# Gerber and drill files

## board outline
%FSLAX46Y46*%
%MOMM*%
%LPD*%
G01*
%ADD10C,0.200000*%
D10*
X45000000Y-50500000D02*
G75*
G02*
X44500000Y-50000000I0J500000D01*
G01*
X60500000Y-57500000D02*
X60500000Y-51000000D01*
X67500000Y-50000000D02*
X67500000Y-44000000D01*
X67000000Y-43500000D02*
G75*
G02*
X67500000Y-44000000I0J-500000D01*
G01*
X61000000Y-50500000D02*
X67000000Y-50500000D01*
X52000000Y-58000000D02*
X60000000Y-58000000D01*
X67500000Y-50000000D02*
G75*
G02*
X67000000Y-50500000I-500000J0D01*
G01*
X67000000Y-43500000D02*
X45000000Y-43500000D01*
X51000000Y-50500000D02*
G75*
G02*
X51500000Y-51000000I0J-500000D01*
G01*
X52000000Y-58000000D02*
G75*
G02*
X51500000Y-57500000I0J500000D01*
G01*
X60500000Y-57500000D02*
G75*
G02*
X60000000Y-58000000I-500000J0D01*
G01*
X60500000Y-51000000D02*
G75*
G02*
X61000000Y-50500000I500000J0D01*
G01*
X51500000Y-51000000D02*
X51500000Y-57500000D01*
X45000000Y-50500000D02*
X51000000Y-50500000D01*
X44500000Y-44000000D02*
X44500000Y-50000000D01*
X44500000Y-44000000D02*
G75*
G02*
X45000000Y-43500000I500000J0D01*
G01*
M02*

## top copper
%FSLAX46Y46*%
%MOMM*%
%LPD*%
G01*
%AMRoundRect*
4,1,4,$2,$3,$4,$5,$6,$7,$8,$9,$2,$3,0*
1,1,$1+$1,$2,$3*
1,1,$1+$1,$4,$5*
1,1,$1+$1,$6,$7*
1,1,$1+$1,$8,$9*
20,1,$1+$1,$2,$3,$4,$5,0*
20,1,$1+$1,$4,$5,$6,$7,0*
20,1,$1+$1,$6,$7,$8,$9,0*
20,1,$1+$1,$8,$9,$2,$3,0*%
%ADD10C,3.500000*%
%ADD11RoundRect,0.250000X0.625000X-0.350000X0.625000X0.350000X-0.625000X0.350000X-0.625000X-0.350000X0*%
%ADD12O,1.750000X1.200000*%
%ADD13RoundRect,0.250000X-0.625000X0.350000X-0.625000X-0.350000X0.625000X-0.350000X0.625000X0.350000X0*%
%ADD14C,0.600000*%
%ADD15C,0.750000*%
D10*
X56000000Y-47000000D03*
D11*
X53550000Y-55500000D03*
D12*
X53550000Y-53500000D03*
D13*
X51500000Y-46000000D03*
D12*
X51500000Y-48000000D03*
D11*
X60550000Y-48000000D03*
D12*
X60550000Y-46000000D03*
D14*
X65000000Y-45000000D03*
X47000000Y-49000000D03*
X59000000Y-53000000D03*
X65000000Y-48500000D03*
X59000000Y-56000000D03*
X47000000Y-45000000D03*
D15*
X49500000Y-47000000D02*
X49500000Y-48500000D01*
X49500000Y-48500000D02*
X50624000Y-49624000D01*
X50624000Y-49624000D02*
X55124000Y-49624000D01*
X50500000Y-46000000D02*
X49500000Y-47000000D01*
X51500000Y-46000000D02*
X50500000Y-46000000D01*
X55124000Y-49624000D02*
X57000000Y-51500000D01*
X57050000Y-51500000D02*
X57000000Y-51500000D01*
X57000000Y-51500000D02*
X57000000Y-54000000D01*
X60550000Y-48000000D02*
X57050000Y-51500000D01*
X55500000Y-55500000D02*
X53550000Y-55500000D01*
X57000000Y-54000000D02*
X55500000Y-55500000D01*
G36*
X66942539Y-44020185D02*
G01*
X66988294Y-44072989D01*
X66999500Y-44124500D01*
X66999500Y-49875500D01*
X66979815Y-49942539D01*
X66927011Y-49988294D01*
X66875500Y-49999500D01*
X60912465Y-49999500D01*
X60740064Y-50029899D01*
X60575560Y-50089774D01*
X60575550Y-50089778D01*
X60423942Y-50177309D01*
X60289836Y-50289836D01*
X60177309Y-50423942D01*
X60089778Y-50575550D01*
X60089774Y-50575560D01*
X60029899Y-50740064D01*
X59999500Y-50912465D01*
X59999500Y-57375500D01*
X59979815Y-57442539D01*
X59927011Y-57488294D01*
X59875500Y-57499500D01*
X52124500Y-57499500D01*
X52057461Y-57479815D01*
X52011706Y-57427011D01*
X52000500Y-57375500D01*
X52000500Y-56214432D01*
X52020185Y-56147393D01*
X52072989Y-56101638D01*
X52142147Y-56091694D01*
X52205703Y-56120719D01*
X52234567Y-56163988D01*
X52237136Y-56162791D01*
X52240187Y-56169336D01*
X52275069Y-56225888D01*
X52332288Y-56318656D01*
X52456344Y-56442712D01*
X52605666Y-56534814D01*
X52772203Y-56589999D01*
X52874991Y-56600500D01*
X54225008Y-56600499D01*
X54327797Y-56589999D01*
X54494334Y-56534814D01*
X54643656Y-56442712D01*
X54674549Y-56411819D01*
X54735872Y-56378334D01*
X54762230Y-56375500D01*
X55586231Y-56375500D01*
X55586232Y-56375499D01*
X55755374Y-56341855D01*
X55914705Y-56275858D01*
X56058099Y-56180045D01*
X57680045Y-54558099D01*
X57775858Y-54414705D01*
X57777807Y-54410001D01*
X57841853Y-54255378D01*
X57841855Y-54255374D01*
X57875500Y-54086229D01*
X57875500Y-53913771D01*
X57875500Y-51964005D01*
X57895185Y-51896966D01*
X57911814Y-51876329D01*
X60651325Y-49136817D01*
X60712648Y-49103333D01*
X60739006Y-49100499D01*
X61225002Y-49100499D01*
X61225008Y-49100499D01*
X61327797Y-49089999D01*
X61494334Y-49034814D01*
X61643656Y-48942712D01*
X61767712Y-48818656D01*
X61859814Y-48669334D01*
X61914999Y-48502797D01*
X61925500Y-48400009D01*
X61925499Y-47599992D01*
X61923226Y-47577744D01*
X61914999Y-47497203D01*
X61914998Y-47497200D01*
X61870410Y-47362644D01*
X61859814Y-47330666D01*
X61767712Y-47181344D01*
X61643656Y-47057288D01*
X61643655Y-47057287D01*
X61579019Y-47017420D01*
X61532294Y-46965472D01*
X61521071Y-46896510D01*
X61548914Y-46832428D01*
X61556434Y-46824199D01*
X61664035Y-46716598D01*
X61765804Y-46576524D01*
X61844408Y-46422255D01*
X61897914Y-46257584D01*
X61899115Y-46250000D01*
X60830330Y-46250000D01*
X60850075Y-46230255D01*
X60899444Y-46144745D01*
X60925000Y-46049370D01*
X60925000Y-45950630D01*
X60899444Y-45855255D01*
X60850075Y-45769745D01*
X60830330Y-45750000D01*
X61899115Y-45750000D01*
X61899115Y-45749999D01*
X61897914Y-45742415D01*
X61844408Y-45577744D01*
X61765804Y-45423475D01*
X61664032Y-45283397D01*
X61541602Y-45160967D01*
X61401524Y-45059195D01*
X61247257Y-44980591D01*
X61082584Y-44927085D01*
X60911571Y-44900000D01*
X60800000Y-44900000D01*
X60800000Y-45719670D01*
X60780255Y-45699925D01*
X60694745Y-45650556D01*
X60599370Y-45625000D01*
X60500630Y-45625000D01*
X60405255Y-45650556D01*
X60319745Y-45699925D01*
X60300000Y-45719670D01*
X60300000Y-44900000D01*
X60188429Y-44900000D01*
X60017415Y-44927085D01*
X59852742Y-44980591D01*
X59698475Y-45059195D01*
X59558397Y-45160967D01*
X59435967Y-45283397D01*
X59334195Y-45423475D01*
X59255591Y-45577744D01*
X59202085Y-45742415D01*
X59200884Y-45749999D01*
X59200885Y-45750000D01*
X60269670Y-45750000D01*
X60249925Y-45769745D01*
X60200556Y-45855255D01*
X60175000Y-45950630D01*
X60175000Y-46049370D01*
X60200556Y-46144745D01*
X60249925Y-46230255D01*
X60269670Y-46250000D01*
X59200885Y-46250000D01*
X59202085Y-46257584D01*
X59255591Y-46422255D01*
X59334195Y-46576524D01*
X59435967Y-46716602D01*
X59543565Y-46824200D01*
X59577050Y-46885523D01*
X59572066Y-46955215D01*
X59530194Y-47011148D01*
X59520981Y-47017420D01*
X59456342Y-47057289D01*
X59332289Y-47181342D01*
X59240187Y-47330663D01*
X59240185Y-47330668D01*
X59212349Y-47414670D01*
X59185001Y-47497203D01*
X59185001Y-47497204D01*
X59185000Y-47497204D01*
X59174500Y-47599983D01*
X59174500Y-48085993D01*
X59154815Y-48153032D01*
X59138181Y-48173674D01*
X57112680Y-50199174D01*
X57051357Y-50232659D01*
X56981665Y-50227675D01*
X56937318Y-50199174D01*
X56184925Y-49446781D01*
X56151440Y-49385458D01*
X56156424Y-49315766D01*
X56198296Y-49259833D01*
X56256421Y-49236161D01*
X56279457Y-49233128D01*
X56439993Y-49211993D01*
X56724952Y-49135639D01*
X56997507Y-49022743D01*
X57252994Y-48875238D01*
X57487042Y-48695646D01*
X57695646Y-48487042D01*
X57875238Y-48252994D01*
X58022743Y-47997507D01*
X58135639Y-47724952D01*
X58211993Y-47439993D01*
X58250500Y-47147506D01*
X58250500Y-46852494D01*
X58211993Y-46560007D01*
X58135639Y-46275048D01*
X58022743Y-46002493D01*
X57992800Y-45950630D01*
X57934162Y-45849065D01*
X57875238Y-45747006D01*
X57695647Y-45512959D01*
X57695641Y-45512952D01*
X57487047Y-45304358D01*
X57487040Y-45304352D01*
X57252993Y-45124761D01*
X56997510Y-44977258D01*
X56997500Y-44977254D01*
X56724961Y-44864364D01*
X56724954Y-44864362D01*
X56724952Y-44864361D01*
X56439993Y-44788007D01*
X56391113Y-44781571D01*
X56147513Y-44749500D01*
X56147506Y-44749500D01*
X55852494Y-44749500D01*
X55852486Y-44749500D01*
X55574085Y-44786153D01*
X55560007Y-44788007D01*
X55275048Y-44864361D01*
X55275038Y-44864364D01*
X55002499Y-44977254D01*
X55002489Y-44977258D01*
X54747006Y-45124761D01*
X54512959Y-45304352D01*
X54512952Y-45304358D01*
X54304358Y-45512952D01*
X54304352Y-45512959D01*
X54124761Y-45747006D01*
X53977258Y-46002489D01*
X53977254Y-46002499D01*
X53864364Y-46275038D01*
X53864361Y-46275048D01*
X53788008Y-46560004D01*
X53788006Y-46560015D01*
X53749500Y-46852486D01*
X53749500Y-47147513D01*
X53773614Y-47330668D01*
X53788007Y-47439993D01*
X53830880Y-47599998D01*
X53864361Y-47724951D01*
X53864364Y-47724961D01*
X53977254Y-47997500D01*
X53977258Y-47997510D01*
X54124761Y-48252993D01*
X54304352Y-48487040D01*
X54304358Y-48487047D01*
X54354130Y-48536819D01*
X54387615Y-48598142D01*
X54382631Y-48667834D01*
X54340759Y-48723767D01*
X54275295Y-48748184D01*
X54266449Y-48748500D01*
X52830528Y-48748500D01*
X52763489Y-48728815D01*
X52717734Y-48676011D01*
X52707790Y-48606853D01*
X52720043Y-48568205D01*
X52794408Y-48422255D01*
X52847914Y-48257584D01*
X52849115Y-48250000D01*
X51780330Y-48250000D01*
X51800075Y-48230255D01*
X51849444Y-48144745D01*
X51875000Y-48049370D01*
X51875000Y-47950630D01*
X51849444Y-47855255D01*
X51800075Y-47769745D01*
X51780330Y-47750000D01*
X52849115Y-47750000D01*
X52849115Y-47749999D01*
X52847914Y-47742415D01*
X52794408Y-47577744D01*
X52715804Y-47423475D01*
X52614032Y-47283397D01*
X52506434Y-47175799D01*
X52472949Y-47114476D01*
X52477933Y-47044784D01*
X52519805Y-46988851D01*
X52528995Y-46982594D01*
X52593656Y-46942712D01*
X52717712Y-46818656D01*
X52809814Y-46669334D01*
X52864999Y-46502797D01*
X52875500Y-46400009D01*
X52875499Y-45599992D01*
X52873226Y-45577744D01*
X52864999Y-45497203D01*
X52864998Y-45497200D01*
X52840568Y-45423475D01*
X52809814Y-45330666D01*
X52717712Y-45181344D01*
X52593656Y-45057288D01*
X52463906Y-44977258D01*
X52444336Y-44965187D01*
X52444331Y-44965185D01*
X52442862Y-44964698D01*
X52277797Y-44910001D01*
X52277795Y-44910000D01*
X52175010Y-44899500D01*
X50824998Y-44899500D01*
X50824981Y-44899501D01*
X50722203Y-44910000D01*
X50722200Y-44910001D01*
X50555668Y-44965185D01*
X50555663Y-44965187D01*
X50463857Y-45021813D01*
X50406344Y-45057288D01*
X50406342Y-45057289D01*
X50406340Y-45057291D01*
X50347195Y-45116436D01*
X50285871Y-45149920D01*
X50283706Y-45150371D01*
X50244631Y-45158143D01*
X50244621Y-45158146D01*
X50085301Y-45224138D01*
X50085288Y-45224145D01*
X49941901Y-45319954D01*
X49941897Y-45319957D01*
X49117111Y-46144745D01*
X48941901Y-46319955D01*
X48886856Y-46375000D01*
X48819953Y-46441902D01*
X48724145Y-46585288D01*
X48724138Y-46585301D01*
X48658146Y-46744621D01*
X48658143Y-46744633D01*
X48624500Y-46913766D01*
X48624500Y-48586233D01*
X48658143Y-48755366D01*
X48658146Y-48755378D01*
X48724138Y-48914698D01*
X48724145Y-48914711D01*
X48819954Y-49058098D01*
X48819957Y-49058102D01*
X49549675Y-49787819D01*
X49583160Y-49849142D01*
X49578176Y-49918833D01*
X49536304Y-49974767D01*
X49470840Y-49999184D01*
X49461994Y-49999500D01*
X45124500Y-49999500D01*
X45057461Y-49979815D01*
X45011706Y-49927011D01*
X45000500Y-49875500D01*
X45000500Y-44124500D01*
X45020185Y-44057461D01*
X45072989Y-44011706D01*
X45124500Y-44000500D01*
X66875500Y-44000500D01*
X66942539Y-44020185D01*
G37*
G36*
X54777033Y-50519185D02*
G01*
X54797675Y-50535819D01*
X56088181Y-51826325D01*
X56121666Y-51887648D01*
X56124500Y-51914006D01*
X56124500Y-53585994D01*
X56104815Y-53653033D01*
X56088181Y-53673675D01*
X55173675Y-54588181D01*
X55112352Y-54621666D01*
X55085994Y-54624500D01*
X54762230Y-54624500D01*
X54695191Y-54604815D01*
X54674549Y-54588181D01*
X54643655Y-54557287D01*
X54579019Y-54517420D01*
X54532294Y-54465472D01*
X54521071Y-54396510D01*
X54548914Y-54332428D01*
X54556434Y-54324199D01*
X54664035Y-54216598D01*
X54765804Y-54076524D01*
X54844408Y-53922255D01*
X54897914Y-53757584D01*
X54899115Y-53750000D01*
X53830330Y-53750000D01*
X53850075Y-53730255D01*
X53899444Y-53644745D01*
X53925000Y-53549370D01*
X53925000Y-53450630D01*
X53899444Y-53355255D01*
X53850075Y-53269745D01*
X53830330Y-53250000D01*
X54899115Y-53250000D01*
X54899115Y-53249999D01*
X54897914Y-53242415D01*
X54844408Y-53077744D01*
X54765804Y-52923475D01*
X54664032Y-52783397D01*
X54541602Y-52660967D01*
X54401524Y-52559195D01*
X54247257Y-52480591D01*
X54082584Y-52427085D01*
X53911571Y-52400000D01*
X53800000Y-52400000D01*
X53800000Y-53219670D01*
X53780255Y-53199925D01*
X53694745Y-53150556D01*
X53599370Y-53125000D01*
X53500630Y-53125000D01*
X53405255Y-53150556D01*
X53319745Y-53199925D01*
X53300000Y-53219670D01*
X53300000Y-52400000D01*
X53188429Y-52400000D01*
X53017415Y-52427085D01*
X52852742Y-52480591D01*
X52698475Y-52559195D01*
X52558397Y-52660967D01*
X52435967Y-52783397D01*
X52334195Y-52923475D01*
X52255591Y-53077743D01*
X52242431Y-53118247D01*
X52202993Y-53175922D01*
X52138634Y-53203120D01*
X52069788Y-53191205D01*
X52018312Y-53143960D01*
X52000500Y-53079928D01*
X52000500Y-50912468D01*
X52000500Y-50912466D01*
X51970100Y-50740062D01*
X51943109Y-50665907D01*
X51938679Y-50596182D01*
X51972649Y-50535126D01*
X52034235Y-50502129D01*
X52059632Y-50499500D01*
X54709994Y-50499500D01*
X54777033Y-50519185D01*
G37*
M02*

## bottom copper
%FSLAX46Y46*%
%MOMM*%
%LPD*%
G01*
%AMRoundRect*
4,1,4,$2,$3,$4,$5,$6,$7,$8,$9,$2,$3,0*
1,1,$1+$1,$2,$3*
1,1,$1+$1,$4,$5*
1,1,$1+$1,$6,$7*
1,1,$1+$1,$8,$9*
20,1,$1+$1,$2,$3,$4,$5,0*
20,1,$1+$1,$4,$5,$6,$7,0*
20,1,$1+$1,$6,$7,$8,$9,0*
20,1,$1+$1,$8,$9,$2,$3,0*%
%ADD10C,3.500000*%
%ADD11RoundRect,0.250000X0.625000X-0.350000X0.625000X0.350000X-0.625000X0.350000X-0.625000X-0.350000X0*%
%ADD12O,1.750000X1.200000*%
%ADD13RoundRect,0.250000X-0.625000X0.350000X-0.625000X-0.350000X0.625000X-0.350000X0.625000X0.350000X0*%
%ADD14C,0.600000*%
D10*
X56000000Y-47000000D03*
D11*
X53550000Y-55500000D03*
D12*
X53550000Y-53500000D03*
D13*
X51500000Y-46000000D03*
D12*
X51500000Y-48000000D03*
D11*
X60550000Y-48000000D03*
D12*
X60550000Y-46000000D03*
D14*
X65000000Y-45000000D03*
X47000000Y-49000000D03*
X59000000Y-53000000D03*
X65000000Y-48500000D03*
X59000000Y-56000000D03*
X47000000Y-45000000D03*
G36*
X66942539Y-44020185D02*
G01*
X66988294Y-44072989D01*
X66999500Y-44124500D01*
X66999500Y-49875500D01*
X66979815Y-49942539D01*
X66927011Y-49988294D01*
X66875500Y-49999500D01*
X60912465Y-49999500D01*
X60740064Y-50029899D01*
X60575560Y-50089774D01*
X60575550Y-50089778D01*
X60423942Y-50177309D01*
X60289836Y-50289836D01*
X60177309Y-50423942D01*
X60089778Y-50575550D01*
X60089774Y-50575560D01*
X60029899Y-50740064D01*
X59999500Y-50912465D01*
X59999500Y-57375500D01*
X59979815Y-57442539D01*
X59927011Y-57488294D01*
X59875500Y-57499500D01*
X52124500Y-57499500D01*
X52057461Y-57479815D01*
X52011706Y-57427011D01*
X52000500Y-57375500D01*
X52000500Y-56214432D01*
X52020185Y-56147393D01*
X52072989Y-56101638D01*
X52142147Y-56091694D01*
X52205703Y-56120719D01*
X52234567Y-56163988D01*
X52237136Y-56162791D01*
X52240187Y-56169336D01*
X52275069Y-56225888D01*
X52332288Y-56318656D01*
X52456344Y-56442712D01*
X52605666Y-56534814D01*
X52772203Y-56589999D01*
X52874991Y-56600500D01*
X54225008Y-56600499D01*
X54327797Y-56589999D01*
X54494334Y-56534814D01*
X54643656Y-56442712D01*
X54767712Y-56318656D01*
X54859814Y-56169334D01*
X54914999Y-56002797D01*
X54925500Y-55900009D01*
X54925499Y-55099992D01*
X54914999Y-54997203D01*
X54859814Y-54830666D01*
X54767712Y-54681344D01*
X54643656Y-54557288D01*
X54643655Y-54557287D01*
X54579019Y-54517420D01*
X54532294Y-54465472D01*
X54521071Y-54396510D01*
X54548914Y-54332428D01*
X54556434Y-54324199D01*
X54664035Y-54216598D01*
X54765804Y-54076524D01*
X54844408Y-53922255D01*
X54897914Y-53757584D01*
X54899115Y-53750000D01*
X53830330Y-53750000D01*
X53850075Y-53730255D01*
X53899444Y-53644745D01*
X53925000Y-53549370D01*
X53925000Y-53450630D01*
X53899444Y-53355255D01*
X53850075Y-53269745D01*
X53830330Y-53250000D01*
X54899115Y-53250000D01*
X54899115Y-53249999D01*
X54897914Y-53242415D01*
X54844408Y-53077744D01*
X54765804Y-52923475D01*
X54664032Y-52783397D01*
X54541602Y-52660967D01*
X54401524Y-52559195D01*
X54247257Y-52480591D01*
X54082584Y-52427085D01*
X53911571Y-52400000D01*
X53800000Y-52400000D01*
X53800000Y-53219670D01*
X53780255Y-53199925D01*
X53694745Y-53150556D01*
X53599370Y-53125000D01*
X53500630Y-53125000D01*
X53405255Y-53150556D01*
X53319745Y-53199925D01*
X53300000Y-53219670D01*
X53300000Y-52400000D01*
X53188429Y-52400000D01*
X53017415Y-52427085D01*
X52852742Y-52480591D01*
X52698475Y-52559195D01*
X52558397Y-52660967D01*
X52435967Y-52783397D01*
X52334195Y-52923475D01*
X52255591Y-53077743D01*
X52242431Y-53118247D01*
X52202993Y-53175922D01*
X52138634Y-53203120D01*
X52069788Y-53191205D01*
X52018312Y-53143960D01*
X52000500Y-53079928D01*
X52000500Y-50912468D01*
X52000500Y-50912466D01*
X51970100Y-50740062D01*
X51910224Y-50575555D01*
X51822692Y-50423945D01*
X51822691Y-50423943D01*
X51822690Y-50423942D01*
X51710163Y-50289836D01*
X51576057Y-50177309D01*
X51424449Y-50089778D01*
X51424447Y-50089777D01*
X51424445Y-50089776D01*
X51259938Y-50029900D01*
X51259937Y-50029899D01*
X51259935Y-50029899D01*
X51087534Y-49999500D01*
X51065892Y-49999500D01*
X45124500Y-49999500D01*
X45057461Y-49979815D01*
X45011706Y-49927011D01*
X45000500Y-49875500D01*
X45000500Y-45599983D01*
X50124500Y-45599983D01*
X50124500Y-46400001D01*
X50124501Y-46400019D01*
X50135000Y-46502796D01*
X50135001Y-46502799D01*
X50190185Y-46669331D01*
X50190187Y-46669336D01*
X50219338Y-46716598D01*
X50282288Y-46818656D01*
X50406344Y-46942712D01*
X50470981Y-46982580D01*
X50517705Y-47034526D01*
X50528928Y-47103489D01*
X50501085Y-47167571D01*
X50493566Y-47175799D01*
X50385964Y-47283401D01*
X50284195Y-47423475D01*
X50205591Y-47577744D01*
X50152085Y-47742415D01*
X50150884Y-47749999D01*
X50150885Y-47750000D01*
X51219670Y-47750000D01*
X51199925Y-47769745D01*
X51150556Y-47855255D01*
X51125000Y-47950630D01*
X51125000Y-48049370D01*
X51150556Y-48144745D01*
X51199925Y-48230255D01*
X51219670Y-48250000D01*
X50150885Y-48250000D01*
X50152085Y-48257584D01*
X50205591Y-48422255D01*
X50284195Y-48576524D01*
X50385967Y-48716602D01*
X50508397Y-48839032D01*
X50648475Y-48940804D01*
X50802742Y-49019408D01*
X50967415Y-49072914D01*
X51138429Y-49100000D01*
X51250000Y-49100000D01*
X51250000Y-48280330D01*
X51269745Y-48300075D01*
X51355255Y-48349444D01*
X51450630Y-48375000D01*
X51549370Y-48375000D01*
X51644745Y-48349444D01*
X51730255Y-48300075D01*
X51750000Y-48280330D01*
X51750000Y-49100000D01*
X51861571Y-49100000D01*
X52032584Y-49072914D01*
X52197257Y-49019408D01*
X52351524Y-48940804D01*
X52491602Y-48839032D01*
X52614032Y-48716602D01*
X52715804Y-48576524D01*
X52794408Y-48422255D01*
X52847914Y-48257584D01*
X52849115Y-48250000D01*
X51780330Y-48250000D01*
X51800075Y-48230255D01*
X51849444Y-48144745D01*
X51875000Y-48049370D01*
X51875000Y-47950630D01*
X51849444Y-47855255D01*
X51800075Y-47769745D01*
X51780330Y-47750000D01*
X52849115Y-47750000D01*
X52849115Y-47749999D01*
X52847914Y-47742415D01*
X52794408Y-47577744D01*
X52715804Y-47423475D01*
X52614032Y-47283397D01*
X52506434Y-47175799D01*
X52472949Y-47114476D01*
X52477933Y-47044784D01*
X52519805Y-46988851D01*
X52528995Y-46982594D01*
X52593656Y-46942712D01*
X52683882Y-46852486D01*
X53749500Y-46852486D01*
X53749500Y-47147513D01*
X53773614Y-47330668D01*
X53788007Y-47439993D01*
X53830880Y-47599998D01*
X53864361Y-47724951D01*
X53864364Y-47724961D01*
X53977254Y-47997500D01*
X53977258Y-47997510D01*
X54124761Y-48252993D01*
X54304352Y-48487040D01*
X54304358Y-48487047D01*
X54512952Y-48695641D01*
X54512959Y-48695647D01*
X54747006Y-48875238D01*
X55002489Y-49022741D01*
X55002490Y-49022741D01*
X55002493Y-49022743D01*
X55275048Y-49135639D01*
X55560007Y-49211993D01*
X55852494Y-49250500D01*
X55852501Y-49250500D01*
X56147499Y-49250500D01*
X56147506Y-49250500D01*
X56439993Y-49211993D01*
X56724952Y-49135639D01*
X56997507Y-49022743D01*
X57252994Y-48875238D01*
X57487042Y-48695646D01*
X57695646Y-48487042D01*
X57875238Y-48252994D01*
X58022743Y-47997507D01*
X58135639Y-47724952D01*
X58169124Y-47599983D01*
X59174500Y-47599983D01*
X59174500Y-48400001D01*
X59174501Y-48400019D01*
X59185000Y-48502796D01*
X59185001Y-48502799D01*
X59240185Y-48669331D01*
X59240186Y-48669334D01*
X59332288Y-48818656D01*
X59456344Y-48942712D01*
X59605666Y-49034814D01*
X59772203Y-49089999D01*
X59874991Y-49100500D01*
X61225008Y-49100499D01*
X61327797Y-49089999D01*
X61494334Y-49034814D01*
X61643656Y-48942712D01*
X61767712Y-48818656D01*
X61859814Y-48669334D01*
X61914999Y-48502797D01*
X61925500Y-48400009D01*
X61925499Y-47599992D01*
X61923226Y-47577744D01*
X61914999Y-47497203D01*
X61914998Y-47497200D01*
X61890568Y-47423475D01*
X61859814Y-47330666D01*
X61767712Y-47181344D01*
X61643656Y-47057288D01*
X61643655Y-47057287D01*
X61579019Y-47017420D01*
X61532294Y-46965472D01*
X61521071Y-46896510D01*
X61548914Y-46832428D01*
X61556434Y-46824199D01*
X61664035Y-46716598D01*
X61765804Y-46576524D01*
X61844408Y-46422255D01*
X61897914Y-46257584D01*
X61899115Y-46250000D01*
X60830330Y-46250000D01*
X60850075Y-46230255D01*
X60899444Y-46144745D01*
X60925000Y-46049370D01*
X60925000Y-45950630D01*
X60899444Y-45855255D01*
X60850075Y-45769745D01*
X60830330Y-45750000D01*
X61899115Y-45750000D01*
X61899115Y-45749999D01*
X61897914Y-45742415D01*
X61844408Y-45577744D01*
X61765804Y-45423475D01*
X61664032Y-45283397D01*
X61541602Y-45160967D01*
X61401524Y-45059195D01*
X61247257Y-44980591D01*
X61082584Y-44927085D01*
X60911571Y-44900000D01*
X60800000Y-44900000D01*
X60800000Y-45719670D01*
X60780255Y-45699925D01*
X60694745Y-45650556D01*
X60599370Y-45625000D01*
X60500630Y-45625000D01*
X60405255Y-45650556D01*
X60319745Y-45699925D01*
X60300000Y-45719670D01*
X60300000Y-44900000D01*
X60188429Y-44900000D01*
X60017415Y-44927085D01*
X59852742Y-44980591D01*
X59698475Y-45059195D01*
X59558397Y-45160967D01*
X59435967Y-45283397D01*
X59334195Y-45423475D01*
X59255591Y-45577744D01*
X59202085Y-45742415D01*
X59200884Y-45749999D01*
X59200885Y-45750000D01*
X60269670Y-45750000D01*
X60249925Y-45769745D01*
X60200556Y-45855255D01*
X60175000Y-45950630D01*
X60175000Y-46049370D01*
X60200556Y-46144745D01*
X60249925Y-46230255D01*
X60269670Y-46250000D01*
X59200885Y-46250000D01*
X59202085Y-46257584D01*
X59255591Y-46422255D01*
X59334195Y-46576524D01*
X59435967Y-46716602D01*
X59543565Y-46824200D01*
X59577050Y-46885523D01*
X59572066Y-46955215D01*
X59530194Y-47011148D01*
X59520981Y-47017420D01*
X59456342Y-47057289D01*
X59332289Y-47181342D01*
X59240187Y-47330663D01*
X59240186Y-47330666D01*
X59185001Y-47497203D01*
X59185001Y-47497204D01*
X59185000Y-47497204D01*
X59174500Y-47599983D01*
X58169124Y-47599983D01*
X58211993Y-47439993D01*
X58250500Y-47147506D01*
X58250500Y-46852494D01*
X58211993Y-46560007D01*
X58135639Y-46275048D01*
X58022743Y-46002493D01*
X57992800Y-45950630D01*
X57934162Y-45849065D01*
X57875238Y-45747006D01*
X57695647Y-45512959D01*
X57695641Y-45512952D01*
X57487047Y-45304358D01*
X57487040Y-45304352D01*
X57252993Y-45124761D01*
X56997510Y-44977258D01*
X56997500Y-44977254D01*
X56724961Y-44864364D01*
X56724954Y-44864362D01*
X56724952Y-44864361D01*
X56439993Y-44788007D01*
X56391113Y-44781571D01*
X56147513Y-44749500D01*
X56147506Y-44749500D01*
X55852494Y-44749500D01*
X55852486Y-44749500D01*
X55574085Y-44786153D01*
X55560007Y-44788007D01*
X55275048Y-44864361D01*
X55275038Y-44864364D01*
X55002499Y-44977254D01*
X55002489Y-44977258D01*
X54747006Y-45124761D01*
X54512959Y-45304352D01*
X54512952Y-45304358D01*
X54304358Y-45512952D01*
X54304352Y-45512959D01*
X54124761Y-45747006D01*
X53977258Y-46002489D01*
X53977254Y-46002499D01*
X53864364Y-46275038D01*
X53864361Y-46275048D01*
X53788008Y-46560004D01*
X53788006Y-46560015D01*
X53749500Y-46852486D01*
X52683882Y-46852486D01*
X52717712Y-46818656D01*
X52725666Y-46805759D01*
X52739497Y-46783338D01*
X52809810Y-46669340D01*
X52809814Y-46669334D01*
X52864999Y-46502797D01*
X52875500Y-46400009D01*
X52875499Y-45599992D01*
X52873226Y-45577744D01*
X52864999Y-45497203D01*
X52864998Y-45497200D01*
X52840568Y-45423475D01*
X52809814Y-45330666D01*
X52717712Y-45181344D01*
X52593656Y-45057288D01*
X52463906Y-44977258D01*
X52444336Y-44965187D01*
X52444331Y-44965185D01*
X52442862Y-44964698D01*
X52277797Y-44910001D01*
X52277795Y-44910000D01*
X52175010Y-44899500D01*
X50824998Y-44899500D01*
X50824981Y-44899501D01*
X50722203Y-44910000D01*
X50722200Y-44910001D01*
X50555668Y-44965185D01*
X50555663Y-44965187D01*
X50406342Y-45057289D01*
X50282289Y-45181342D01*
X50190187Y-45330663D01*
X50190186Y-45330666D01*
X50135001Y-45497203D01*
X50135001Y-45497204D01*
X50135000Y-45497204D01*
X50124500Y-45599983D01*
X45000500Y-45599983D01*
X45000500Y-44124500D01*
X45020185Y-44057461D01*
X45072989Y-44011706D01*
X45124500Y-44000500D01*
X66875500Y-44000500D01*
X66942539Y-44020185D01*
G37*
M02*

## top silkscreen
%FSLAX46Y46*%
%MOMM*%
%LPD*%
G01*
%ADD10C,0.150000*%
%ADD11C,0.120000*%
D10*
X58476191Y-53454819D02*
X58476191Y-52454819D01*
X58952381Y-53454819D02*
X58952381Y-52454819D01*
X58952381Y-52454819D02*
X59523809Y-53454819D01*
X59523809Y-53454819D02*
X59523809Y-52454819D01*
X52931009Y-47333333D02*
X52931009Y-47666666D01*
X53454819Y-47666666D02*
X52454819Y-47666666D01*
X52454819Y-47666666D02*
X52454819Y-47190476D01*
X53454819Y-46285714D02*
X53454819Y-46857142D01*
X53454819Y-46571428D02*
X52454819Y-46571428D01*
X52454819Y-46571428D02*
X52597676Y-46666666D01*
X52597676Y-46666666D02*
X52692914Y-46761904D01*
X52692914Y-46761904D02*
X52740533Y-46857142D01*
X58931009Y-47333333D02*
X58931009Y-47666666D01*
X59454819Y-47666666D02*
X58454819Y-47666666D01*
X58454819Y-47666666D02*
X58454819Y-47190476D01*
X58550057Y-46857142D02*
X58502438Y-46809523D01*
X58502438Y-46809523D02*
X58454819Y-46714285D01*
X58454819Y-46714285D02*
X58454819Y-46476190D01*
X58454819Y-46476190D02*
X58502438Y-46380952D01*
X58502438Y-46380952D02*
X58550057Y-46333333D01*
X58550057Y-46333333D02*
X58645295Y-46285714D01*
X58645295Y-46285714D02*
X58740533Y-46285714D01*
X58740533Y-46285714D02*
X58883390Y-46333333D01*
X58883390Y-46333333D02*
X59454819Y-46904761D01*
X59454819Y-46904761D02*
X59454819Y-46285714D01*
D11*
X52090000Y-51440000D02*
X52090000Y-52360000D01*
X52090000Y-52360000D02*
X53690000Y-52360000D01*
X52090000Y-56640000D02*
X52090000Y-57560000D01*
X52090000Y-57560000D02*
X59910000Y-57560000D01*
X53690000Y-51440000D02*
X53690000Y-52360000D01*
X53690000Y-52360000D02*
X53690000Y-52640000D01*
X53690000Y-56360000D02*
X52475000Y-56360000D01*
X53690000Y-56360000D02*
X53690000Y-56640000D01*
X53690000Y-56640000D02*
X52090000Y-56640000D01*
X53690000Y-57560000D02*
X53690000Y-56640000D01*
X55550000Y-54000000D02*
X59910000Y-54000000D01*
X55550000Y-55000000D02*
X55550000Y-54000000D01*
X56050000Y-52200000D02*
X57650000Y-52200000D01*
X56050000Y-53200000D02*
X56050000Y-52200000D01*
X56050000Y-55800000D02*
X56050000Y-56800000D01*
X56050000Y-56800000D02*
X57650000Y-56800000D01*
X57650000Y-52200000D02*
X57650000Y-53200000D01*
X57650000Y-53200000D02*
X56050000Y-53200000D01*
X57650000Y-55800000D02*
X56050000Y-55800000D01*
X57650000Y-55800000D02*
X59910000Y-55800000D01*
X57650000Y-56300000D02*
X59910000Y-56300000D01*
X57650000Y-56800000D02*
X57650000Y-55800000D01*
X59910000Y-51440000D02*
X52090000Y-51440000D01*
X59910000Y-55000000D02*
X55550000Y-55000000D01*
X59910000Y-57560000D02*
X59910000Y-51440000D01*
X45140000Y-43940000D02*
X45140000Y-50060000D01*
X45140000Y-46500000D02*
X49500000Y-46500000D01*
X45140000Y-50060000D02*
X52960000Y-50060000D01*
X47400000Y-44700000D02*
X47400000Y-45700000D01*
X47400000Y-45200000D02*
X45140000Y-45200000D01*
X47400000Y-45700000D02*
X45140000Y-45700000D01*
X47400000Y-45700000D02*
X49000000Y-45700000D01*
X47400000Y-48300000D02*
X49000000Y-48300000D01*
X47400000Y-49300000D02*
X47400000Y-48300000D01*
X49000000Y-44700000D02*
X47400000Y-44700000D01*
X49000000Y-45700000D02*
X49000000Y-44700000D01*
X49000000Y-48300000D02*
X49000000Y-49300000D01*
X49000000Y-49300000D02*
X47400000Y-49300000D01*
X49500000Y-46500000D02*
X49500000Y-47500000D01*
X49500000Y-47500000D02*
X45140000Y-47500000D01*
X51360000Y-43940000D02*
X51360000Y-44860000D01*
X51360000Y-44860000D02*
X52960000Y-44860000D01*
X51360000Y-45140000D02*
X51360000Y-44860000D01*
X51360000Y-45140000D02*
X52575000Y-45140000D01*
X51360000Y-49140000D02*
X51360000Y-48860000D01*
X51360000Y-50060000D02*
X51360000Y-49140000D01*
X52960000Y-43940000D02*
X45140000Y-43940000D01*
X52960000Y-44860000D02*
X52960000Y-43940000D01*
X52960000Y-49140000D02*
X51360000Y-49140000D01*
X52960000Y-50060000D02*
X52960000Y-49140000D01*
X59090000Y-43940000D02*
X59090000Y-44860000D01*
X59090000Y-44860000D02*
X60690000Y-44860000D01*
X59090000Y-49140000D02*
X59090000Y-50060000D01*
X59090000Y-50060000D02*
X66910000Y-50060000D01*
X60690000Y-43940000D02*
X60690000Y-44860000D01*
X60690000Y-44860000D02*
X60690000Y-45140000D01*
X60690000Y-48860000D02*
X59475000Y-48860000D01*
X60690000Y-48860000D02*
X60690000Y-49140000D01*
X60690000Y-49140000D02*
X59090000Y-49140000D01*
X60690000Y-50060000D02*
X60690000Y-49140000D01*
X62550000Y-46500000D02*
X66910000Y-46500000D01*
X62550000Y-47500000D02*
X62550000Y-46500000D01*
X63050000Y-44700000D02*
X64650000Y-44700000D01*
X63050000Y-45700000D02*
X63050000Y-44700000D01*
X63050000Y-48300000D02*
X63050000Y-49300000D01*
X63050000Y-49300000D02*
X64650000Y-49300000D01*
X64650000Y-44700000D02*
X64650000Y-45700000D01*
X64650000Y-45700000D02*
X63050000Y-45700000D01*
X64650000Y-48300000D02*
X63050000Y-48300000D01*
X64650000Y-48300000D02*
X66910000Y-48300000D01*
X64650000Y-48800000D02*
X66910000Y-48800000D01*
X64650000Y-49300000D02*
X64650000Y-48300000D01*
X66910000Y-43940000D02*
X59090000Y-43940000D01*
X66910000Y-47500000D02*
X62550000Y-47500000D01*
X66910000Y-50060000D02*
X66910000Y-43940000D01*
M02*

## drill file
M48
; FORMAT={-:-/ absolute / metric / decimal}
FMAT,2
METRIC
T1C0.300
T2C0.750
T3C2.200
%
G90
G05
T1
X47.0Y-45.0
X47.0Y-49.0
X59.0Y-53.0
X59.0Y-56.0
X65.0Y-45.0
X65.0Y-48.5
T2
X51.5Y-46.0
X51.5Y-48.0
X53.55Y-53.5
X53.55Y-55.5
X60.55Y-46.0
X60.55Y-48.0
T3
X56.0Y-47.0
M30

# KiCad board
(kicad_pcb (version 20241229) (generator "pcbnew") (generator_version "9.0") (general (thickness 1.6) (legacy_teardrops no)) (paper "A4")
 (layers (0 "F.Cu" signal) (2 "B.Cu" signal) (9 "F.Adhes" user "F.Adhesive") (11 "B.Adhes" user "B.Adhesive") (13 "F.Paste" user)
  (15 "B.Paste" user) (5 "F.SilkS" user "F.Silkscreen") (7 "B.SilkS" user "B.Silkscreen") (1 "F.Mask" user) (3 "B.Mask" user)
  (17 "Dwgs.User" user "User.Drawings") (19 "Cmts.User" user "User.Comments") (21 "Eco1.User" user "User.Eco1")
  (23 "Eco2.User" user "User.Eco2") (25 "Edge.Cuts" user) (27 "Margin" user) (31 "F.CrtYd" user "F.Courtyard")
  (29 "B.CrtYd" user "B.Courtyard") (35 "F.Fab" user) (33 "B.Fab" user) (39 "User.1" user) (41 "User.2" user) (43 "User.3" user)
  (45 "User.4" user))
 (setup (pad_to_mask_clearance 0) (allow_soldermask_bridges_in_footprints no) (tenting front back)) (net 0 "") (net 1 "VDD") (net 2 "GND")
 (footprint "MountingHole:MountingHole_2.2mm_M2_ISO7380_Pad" (layer "F.Cu") (at 56 47)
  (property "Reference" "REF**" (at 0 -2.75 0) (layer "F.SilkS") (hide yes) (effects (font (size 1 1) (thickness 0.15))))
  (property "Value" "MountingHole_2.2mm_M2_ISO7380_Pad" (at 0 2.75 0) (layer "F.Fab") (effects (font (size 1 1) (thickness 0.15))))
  (pad "1" thru_hole circle (at 0 0) (size 3.5 3.5) (drill 2.2) (layers "*.Cu" "*.Mask") (remove_unused_layers no)))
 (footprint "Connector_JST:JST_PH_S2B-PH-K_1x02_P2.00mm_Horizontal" (layer "F.Cu") (at 53.55 55.5 90)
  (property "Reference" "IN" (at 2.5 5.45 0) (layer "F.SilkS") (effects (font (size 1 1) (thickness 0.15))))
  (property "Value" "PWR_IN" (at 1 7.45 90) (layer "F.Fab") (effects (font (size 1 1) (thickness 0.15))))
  (fp_line (start 4.06 -1.46) (end 3.14 -1.46) (stroke (width 0.12) (type solid)) (layer "F.SilkS"))
  (fp_line (start 3.14 -1.46) (end 3.14 0.14) (stroke (width 0.12) (type solid)) (layer "F.SilkS"))
  (fp_line (start -1.14 -1.46) (end -2.06 -1.46) (stroke (width 0.12) (type solid)) (layer "F.SilkS"))
  (fp_line (start -2.06 -1.46) (end -2.06 6.36) (stroke (width 0.12) (type solid)) (layer "F.SilkS"))
  (fp_line (start 4.06 0.14) (end 3.14 0.14) (stroke (width 0.12) (type solid)) (layer "F.SilkS"))
  (fp_line (start 3.14 0.14) (end 2.86 0.14) (stroke (width 0.12) (type solid)) (layer "F.SilkS"))
  (fp_line (start -0.86 0.14) (end -0.86 -1.075) (stroke (width 0.12) (type solid)) (layer "F.SilkS"))
  (fp_line (start -0.86 0.14) (end -1.14 0.14) (stroke (width 0.12) (type solid)) (layer "F.SilkS"))
  (fp_line (start -1.14 0.14) (end -1.14 -1.46) (stroke (width 0.12) (type solid)) (layer "F.SilkS"))
  (fp_line (start -2.06 0.14) (end -1.14 0.14) (stroke (width 0.12) (type solid)) (layer "F.SilkS"))
  (fp_line (start 1.5 2) (end 1.5 6.36) (stroke (width 0.12) (type solid)) (layer "F.SilkS"))
  (fp_line (start 0.5 2) (end 1.5 2) (stroke (width 0.12) (type solid)) (layer "F.SilkS"))
  (fp_line (start 3.3 2.5) (end 3.3 4.1) (stroke (width 0.12) (type solid)) (layer "F.SilkS"))
  (fp_line (start 2.3 2.5) (end 3.3 2.5) (stroke (width 0.12) (type solid)) (layer "F.SilkS"))
  (fp_line (start -0.3 2.5) (end -1.3 2.5) (stroke (width 0.12) (type solid)) (layer "F.SilkS"))
  (fp_line (start -1.3 2.5) (end -1.3 4.1) (stroke (width 0.12) (type solid)) (layer "F.SilkS"))
  (fp_line (start 3.3 4.1) (end 2.3 4.1) (stroke (width 0.12) (type solid)) (layer "F.SilkS"))
  (fp_line (start 2.3 4.1) (end 2.3 2.5) (stroke (width 0.12) (type solid)) (layer "F.SilkS"))
  (fp_line (start -0.3 4.1) (end -0.3 2.5) (stroke (width 0.12) (type solid)) (layer "F.SilkS"))
  (fp_line (start -0.3 4.1) (end -0.3 6.36) (stroke (width 0.12) (type solid)) (layer "F.SilkS"))
  (fp_line (start -0.8 4.1) (end -0.8 6.36) (stroke (width 0.12) (type solid)) (layer "F.SilkS"))
  (fp_line (start -1.3 4.1) (end -0.3 4.1) (stroke (width 0.12) (type solid)) (layer "F.SilkS"))
  (fp_line (start 4.06 6.36) (end 4.06 -1.46) (stroke (width 0.12) (type solid)) (layer "F.SilkS"))
  (fp_line (start 0.5 6.36) (end 0.5 2) (stroke (width 0.12) (type solid)) (layer "F.SilkS"))
  (fp_line (start -2.06 6.36) (end 4.06 6.36) (stroke (width 0.12) (type solid)) (layer "F.SilkS"))
  (pad "1" thru_hole roundrect (at 0 0 90) (size 1.2 1.75) (drill 0.75) (layers "*.Cu" "*.Mask") (remove_unused_layers no)
   (roundrect_rratio 0.208333) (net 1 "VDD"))
  (pad "2" thru_hole oval (at 2 0 90) (size 1.2 1.75) (drill 0.75) (layers "*.Cu" "*.Mask") (remove_unused_layers no) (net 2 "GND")))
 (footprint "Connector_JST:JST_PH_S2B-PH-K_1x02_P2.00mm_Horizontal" (layer "F.Cu") (at 51.5 46 -90)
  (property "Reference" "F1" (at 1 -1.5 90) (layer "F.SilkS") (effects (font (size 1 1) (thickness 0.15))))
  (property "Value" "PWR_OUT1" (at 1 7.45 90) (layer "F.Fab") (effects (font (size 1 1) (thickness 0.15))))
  (fp_line (start -2.06 6.36) (end 4.06 6.36) (stroke (width 0.12) (type solid)) (layer "F.SilkS"))
  (fp_line (start 0.5 6.36) (end 0.5 2) (stroke (width 0.12) (type solid)) (layer "F.SilkS"))
  (fp_line (start 4.06 6.36) (end 4.06 -1.46) (stroke (width 0.12) (type solid)) (layer "F.SilkS"))
  (fp_line (start -1.3 4.1) (end -0.3 4.1) (stroke (width 0.12) (type solid)) (layer "F.SilkS"))
  (fp_line (start -0.8 4.1) (end -0.8 6.36) (stroke (width 0.12) (type solid)) (layer "F.SilkS"))
  (fp_line (start -0.3 4.1) (end -0.3 6.36) (stroke (width 0.12) (type solid)) (layer "F.SilkS"))
  (fp_line (start -0.3 4.1) (end -0.3 2.5) (stroke (width 0.12) (type solid)) (layer "F.SilkS"))
  (fp_line (start 2.3 4.1) (end 2.3 2.5) (stroke (width 0.12) (type solid)) (layer "F.SilkS"))
  (fp_line (start 3.3 4.1) (end 2.3 4.1) (stroke (width 0.12) (type solid)) (layer "F.SilkS"))
  (fp_line (start -1.3 2.5) (end -1.3 4.1) (stroke (width 0.12) (type solid)) (layer "F.SilkS"))
  (fp_line (start -0.3 2.5) (end -1.3 2.5) (stroke (width 0.12) (type solid)) (layer "F.SilkS"))
  (fp_line (start 2.3 2.5) (end 3.3 2.5) (stroke (width 0.12) (type solid)) (layer "F.SilkS"))
  (fp_line (start 3.3 2.5) (end 3.3 4.1) (stroke (width 0.12) (type solid)) (layer "F.SilkS"))
  (fp_line (start 0.5 2) (end 1.5 2) (stroke (width 0.12) (type solid)) (layer "F.SilkS"))
  (fp_line (start 1.5 2) (end 1.5 6.36) (stroke (width 0.12) (type solid)) (layer "F.SilkS"))
  (fp_line (start -2.06 0.14) (end -1.14 0.14) (stroke (width 0.12) (type solid)) (layer "F.SilkS"))
  (fp_line (start -1.14 0.14) (end -1.14 -1.46) (stroke (width 0.12) (type solid)) (layer "F.SilkS"))
  (fp_line (start -0.86 0.14) (end -1.14 0.14) (stroke (width 0.12) (type solid)) (layer "F.SilkS"))
  (fp_line (start -0.86 0.14) (end -0.86 -1.075) (stroke (width 0.12) (type solid)) (layer "F.SilkS"))
  (fp_line (start 3.14 0.14) (end 2.86 0.14) (stroke (width 0.12) (type solid)) (layer "F.SilkS"))
  (fp_line (start 4.06 0.14) (end 3.14 0.14) (stroke (width 0.12) (type solid)) (layer "F.SilkS"))
  (fp_line (start -2.06 -1.46) (end -2.06 6.36) (stroke (width 0.12) (type solid)) (layer "F.SilkS"))
  (fp_line (start -1.14 -1.46) (end -2.06 -1.46) (stroke (width 0.12) (type solid)) (layer "F.SilkS"))
  (fp_line (start 3.14 -1.46) (end 3.14 0.14) (stroke (width 0.12) (type solid)) (layer "F.SilkS"))
  (fp_line (start 4.06 -1.46) (end 3.14 -1.46) (stroke (width 0.12) (type solid)) (layer "F.SilkS"))
  (pad "1" thru_hole roundrect (at 0 0 270) (size 1.2 1.75) (drill 0.75) (layers "*.Cu" "*.Mask") (remove_unused_layers no)
   (roundrect_rratio 0.208333) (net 1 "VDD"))
  (pad "2" thru_hole oval (at 2 0 270) (size 1.2 1.75) (drill 0.75) (layers "*.Cu" "*.Mask") (remove_unused_layers no) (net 2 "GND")))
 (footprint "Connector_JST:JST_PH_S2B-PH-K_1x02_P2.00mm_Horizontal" (layer "F.Cu") (at 60.55 48 90)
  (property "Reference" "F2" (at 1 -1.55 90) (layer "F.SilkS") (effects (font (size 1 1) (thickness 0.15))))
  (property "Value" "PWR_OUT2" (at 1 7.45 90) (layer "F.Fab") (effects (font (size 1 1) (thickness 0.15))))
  (fp_line (start 4.06 -1.46) (end 3.14 -1.46) (stroke (width 0.12) (type solid)) (layer "F.SilkS"))
  (fp_line (start 3.14 -1.46) (end 3.14 0.14) (stroke (width 0.12) (type solid)) (layer "F.SilkS"))
  (fp_line (start -1.14 -1.46) (end -2.06 -1.46) (stroke (width 0.12) (type solid)) (layer "F.SilkS"))
  (fp_line (start -2.06 -1.46) (end -2.06 6.36) (stroke (width 0.12) (type solid)) (layer "F.SilkS"))
  (fp_line (start 4.06 0.14) (end 3.14 0.14) (stroke (width 0.12) (type solid)) (layer "F.SilkS"))
  (fp_line (start 3.14 0.14) (end 2.86 0.14) (stroke (width 0.12) (type solid)) (layer "F.SilkS"))
  (fp_line (start -0.86 0.14) (end -0.86 -1.075) (stroke (width 0.12) (type solid)) (layer "F.SilkS"))
  (fp_line (start -0.86 0.14) (end -1.14 0.14) (stroke (width 0.12) (type solid)) (layer "F.SilkS"))
  (fp_line (start -1.14 0.14) (end -1.14 -1.46) (stroke (width 0.12) (type solid)) (layer "F.SilkS"))
  (fp_line (start -2.06 0.14) (end -1.14 0.14) (stroke (width 0.12) (type solid)) (layer "F.SilkS"))
  (fp_line (start 1.5 2) (end 1.5 6.36) (stroke (width 0.12) (type solid)) (layer "F.SilkS"))
  (fp_line (start 0.5 2) (end 1.5 2) (stroke (width 0.12) (type solid)) (layer "F.SilkS"))
  (fp_line (start 3.3 2.5) (end 3.3 4.1) (stroke (width 0.12) (type solid)) (layer "F.SilkS"))
  (fp_line (start 2.3 2.5) (end 3.3 2.5) (stroke (width 0.12) (type solid)) (layer "F.SilkS"))
  (fp_line (start -0.3 2.5) (end -1.3 2.5) (stroke (width 0.12) (type solid)) (layer "F.SilkS"))
  (fp_line (start -1.3 2.5) (end -1.3 4.1) (stroke (width 0.12) (type solid)) (layer "F.SilkS"))
  (fp_line (start 3.3 4.1) (end 2.3 4.1) (stroke (width 0.12) (type solid)) (layer "F.SilkS"))
  (fp_line (start 2.3 4.1) (end 2.3 2.5) (stroke (width 0.12) (type solid)) (layer "F.SilkS"))
  (fp_line (start -0.3 4.1) (end -0.3 2.5) (stroke (width 0.12) (type solid)) (layer "F.SilkS"))
  (fp_line (start -0.3 4.1) (end -0.3 6.36) (stroke (width 0.12) (type solid)) (layer "F.SilkS"))
  (fp_line (start -0.8 4.1) (end -0.8 6.36) (stroke (width 0.12) (type solid)) (layer "F.SilkS"))
  (fp_line (start -1.3 4.1) (end -0.3 4.1) (stroke (width 0.12) (type solid)) (layer "F.SilkS"))
  (fp_line (start 4.06 6.36) (end 4.06 -1.46) (stroke (width 0.12) (type solid)) (layer "F.SilkS"))
  (fp_line (start 0.5 6.36) (end 0.5 2) (stroke (width 0.12) (type solid)) (layer "F.SilkS"))
  (fp_line (start -2.06 6.36) (end 4.06 6.36) (stroke (width 0.12) (type solid)) (layer "F.SilkS"))
  (pad "1" thru_hole roundrect (at 0 0 90) (size 1.2 1.75) (drill 0.75) (layers "*.Cu" "*.Mask") (remove_unused_layers no)
   (roundrect_rratio 0.208333) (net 1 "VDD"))
  (pad "2" thru_hole oval (at 2 0 90) (size 1.2 1.75) (drill 0.75) (layers "*.Cu" "*.Mask") (remove_unused_layers no) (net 2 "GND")))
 (gr_arc (start 45 50.5) (mid 44.646447 50.353553) (end 44.5 50) (stroke (width 0.2) (type default)) (layer "Edge.Cuts"))
 (gr_line (start 60.5 57.5) (end 60.5 51) (stroke (width 0.2) (type default)) (layer "Edge.Cuts"))
 (gr_line (start 67.5 50) (end 67.5 44) (stroke (width 0.2) (type default)) (layer "Edge.Cuts"))
 (gr_arc (start 67 43.5) (mid 67.353553 43.646447) (end 67.5 44) (stroke (width 0.2) (type default)) (layer "Edge.Cuts"))
 (gr_line (start 61 50.5) (end 67 50.5) (stroke (width 0.2) (type default)) (layer "Edge.Cuts"))
 (gr_line (start 52 58) (end 60 58) (stroke (width 0.2) (type default)) (layer "Edge.Cuts"))
 (gr_arc (start 67.5 50) (mid 67.353553 50.353553) (end 67 50.5) (stroke (width 0.2) (type default)) (layer "Edge.Cuts"))
 (gr_line (start 67 43.5) (end 45 43.5) (stroke (width 0.2) (type default)) (layer "Edge.Cuts"))
 (gr_arc (start 51 50.5) (mid 51.353553 50.646447) (end 51.5 51) (stroke (width 0.2) (type default)) (layer "Edge.Cuts"))
 (gr_arc (start 52 58) (mid 51.646447 57.853553) (end 51.5 57.5) (stroke (width 0.2) (type default)) (layer "Edge.Cuts"))
 (gr_arc (start 60.5 57.5) (mid 60.353553 57.853553) (end 60 58) (stroke (width 0.2) (type default)) (layer "Edge.Cuts"))
 (gr_arc (start 60.5 51) (mid 60.646447 50.646447) (end 61 50.5) (stroke (width 0.2) (type default)) (layer "Edge.Cuts"))
 (gr_line (start 51.5 51) (end 51.5 57.5) (stroke (width 0.2) (type default)) (layer "Edge.Cuts"))
 (gr_line (start 45 50.5) (end 51 50.5) (stroke (width 0.2) (type default)) (layer "Edge.Cuts"))
 (gr_line (start 44.5 44) (end 44.5 50) (stroke (width 0.2) (type default)) (layer "Edge.Cuts"))
 (gr_arc (start 44.5 44) (mid 44.646447 43.646447) (end 45 43.5) (stroke (width 0.2) (type default)) (layer "Edge.Cuts"))
 (segment (start 49.5 47) (end 49.5 48.5) (width 0.75) (layer "F.Cu") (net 1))
 (segment (start 49.5 48.5) (end 50.624 49.624) (width 0.75) (layer "F.Cu") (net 1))
 (segment (start 50.624 49.624) (end 55.124 49.624) (width 0.75) (layer "F.Cu") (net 1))
 (segment (start 50.5 46) (end 49.5 47) (width 0.75) (layer "F.Cu") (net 1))
 (segment (start 51.5 46) (end 50.5 46) (width 0.75) (layer "F.Cu") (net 1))
 (segment (start 55.124 49.624) (end 57 51.5) (width 0.75) (layer "F.Cu") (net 1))
 (segment (start 57.05 51.5) (end 57 51.5) (width 0.75) (layer "F.Cu") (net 1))
 (segment (start 57 51.5) (end 57 54) (width 0.75) (layer "F.Cu") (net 1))
 (segment (start 60.55 48) (end 57.05 51.5) (width 0.75) (layer "F.Cu") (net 1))
 (segment (start 55.5 55.5) (end 53.55 55.5) (width 0.75) (layer "F.Cu") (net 1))
 (segment (start 57 54) (end 55.5 55.5) (width 0.75) (layer "F.Cu") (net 1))
 (via (at 65 45) (size 0.6) (drill 0.3) (layers "F.Cu" "B.Cu") (free yes) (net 2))
 (via (at 47 49) (size 0.6) (drill 0.3) (layers "F.Cu" "B.Cu") (free yes) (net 2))
 (via (at 59 53) (size 0.6) (drill 0.3) (layers "F.Cu" "B.Cu") (free yes) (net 2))
 (via (at 65 48.5) (size 0.6) (drill 0.3) (layers "F.Cu" "B.Cu") (free yes) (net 2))
 (via (at 59 56) (size 0.6) (drill 0.3) (layers "F.Cu" "B.Cu") (free yes) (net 2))
 (via (at 47 45) (size 0.6) (drill 0.3) (layers "F.Cu" "B.Cu") (free yes) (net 2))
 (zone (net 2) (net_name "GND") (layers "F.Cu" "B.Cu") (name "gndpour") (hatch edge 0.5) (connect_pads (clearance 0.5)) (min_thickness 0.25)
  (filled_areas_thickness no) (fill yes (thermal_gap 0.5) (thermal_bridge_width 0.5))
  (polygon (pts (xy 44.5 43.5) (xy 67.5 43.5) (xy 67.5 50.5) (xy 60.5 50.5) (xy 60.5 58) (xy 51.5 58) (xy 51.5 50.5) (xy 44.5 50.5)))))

